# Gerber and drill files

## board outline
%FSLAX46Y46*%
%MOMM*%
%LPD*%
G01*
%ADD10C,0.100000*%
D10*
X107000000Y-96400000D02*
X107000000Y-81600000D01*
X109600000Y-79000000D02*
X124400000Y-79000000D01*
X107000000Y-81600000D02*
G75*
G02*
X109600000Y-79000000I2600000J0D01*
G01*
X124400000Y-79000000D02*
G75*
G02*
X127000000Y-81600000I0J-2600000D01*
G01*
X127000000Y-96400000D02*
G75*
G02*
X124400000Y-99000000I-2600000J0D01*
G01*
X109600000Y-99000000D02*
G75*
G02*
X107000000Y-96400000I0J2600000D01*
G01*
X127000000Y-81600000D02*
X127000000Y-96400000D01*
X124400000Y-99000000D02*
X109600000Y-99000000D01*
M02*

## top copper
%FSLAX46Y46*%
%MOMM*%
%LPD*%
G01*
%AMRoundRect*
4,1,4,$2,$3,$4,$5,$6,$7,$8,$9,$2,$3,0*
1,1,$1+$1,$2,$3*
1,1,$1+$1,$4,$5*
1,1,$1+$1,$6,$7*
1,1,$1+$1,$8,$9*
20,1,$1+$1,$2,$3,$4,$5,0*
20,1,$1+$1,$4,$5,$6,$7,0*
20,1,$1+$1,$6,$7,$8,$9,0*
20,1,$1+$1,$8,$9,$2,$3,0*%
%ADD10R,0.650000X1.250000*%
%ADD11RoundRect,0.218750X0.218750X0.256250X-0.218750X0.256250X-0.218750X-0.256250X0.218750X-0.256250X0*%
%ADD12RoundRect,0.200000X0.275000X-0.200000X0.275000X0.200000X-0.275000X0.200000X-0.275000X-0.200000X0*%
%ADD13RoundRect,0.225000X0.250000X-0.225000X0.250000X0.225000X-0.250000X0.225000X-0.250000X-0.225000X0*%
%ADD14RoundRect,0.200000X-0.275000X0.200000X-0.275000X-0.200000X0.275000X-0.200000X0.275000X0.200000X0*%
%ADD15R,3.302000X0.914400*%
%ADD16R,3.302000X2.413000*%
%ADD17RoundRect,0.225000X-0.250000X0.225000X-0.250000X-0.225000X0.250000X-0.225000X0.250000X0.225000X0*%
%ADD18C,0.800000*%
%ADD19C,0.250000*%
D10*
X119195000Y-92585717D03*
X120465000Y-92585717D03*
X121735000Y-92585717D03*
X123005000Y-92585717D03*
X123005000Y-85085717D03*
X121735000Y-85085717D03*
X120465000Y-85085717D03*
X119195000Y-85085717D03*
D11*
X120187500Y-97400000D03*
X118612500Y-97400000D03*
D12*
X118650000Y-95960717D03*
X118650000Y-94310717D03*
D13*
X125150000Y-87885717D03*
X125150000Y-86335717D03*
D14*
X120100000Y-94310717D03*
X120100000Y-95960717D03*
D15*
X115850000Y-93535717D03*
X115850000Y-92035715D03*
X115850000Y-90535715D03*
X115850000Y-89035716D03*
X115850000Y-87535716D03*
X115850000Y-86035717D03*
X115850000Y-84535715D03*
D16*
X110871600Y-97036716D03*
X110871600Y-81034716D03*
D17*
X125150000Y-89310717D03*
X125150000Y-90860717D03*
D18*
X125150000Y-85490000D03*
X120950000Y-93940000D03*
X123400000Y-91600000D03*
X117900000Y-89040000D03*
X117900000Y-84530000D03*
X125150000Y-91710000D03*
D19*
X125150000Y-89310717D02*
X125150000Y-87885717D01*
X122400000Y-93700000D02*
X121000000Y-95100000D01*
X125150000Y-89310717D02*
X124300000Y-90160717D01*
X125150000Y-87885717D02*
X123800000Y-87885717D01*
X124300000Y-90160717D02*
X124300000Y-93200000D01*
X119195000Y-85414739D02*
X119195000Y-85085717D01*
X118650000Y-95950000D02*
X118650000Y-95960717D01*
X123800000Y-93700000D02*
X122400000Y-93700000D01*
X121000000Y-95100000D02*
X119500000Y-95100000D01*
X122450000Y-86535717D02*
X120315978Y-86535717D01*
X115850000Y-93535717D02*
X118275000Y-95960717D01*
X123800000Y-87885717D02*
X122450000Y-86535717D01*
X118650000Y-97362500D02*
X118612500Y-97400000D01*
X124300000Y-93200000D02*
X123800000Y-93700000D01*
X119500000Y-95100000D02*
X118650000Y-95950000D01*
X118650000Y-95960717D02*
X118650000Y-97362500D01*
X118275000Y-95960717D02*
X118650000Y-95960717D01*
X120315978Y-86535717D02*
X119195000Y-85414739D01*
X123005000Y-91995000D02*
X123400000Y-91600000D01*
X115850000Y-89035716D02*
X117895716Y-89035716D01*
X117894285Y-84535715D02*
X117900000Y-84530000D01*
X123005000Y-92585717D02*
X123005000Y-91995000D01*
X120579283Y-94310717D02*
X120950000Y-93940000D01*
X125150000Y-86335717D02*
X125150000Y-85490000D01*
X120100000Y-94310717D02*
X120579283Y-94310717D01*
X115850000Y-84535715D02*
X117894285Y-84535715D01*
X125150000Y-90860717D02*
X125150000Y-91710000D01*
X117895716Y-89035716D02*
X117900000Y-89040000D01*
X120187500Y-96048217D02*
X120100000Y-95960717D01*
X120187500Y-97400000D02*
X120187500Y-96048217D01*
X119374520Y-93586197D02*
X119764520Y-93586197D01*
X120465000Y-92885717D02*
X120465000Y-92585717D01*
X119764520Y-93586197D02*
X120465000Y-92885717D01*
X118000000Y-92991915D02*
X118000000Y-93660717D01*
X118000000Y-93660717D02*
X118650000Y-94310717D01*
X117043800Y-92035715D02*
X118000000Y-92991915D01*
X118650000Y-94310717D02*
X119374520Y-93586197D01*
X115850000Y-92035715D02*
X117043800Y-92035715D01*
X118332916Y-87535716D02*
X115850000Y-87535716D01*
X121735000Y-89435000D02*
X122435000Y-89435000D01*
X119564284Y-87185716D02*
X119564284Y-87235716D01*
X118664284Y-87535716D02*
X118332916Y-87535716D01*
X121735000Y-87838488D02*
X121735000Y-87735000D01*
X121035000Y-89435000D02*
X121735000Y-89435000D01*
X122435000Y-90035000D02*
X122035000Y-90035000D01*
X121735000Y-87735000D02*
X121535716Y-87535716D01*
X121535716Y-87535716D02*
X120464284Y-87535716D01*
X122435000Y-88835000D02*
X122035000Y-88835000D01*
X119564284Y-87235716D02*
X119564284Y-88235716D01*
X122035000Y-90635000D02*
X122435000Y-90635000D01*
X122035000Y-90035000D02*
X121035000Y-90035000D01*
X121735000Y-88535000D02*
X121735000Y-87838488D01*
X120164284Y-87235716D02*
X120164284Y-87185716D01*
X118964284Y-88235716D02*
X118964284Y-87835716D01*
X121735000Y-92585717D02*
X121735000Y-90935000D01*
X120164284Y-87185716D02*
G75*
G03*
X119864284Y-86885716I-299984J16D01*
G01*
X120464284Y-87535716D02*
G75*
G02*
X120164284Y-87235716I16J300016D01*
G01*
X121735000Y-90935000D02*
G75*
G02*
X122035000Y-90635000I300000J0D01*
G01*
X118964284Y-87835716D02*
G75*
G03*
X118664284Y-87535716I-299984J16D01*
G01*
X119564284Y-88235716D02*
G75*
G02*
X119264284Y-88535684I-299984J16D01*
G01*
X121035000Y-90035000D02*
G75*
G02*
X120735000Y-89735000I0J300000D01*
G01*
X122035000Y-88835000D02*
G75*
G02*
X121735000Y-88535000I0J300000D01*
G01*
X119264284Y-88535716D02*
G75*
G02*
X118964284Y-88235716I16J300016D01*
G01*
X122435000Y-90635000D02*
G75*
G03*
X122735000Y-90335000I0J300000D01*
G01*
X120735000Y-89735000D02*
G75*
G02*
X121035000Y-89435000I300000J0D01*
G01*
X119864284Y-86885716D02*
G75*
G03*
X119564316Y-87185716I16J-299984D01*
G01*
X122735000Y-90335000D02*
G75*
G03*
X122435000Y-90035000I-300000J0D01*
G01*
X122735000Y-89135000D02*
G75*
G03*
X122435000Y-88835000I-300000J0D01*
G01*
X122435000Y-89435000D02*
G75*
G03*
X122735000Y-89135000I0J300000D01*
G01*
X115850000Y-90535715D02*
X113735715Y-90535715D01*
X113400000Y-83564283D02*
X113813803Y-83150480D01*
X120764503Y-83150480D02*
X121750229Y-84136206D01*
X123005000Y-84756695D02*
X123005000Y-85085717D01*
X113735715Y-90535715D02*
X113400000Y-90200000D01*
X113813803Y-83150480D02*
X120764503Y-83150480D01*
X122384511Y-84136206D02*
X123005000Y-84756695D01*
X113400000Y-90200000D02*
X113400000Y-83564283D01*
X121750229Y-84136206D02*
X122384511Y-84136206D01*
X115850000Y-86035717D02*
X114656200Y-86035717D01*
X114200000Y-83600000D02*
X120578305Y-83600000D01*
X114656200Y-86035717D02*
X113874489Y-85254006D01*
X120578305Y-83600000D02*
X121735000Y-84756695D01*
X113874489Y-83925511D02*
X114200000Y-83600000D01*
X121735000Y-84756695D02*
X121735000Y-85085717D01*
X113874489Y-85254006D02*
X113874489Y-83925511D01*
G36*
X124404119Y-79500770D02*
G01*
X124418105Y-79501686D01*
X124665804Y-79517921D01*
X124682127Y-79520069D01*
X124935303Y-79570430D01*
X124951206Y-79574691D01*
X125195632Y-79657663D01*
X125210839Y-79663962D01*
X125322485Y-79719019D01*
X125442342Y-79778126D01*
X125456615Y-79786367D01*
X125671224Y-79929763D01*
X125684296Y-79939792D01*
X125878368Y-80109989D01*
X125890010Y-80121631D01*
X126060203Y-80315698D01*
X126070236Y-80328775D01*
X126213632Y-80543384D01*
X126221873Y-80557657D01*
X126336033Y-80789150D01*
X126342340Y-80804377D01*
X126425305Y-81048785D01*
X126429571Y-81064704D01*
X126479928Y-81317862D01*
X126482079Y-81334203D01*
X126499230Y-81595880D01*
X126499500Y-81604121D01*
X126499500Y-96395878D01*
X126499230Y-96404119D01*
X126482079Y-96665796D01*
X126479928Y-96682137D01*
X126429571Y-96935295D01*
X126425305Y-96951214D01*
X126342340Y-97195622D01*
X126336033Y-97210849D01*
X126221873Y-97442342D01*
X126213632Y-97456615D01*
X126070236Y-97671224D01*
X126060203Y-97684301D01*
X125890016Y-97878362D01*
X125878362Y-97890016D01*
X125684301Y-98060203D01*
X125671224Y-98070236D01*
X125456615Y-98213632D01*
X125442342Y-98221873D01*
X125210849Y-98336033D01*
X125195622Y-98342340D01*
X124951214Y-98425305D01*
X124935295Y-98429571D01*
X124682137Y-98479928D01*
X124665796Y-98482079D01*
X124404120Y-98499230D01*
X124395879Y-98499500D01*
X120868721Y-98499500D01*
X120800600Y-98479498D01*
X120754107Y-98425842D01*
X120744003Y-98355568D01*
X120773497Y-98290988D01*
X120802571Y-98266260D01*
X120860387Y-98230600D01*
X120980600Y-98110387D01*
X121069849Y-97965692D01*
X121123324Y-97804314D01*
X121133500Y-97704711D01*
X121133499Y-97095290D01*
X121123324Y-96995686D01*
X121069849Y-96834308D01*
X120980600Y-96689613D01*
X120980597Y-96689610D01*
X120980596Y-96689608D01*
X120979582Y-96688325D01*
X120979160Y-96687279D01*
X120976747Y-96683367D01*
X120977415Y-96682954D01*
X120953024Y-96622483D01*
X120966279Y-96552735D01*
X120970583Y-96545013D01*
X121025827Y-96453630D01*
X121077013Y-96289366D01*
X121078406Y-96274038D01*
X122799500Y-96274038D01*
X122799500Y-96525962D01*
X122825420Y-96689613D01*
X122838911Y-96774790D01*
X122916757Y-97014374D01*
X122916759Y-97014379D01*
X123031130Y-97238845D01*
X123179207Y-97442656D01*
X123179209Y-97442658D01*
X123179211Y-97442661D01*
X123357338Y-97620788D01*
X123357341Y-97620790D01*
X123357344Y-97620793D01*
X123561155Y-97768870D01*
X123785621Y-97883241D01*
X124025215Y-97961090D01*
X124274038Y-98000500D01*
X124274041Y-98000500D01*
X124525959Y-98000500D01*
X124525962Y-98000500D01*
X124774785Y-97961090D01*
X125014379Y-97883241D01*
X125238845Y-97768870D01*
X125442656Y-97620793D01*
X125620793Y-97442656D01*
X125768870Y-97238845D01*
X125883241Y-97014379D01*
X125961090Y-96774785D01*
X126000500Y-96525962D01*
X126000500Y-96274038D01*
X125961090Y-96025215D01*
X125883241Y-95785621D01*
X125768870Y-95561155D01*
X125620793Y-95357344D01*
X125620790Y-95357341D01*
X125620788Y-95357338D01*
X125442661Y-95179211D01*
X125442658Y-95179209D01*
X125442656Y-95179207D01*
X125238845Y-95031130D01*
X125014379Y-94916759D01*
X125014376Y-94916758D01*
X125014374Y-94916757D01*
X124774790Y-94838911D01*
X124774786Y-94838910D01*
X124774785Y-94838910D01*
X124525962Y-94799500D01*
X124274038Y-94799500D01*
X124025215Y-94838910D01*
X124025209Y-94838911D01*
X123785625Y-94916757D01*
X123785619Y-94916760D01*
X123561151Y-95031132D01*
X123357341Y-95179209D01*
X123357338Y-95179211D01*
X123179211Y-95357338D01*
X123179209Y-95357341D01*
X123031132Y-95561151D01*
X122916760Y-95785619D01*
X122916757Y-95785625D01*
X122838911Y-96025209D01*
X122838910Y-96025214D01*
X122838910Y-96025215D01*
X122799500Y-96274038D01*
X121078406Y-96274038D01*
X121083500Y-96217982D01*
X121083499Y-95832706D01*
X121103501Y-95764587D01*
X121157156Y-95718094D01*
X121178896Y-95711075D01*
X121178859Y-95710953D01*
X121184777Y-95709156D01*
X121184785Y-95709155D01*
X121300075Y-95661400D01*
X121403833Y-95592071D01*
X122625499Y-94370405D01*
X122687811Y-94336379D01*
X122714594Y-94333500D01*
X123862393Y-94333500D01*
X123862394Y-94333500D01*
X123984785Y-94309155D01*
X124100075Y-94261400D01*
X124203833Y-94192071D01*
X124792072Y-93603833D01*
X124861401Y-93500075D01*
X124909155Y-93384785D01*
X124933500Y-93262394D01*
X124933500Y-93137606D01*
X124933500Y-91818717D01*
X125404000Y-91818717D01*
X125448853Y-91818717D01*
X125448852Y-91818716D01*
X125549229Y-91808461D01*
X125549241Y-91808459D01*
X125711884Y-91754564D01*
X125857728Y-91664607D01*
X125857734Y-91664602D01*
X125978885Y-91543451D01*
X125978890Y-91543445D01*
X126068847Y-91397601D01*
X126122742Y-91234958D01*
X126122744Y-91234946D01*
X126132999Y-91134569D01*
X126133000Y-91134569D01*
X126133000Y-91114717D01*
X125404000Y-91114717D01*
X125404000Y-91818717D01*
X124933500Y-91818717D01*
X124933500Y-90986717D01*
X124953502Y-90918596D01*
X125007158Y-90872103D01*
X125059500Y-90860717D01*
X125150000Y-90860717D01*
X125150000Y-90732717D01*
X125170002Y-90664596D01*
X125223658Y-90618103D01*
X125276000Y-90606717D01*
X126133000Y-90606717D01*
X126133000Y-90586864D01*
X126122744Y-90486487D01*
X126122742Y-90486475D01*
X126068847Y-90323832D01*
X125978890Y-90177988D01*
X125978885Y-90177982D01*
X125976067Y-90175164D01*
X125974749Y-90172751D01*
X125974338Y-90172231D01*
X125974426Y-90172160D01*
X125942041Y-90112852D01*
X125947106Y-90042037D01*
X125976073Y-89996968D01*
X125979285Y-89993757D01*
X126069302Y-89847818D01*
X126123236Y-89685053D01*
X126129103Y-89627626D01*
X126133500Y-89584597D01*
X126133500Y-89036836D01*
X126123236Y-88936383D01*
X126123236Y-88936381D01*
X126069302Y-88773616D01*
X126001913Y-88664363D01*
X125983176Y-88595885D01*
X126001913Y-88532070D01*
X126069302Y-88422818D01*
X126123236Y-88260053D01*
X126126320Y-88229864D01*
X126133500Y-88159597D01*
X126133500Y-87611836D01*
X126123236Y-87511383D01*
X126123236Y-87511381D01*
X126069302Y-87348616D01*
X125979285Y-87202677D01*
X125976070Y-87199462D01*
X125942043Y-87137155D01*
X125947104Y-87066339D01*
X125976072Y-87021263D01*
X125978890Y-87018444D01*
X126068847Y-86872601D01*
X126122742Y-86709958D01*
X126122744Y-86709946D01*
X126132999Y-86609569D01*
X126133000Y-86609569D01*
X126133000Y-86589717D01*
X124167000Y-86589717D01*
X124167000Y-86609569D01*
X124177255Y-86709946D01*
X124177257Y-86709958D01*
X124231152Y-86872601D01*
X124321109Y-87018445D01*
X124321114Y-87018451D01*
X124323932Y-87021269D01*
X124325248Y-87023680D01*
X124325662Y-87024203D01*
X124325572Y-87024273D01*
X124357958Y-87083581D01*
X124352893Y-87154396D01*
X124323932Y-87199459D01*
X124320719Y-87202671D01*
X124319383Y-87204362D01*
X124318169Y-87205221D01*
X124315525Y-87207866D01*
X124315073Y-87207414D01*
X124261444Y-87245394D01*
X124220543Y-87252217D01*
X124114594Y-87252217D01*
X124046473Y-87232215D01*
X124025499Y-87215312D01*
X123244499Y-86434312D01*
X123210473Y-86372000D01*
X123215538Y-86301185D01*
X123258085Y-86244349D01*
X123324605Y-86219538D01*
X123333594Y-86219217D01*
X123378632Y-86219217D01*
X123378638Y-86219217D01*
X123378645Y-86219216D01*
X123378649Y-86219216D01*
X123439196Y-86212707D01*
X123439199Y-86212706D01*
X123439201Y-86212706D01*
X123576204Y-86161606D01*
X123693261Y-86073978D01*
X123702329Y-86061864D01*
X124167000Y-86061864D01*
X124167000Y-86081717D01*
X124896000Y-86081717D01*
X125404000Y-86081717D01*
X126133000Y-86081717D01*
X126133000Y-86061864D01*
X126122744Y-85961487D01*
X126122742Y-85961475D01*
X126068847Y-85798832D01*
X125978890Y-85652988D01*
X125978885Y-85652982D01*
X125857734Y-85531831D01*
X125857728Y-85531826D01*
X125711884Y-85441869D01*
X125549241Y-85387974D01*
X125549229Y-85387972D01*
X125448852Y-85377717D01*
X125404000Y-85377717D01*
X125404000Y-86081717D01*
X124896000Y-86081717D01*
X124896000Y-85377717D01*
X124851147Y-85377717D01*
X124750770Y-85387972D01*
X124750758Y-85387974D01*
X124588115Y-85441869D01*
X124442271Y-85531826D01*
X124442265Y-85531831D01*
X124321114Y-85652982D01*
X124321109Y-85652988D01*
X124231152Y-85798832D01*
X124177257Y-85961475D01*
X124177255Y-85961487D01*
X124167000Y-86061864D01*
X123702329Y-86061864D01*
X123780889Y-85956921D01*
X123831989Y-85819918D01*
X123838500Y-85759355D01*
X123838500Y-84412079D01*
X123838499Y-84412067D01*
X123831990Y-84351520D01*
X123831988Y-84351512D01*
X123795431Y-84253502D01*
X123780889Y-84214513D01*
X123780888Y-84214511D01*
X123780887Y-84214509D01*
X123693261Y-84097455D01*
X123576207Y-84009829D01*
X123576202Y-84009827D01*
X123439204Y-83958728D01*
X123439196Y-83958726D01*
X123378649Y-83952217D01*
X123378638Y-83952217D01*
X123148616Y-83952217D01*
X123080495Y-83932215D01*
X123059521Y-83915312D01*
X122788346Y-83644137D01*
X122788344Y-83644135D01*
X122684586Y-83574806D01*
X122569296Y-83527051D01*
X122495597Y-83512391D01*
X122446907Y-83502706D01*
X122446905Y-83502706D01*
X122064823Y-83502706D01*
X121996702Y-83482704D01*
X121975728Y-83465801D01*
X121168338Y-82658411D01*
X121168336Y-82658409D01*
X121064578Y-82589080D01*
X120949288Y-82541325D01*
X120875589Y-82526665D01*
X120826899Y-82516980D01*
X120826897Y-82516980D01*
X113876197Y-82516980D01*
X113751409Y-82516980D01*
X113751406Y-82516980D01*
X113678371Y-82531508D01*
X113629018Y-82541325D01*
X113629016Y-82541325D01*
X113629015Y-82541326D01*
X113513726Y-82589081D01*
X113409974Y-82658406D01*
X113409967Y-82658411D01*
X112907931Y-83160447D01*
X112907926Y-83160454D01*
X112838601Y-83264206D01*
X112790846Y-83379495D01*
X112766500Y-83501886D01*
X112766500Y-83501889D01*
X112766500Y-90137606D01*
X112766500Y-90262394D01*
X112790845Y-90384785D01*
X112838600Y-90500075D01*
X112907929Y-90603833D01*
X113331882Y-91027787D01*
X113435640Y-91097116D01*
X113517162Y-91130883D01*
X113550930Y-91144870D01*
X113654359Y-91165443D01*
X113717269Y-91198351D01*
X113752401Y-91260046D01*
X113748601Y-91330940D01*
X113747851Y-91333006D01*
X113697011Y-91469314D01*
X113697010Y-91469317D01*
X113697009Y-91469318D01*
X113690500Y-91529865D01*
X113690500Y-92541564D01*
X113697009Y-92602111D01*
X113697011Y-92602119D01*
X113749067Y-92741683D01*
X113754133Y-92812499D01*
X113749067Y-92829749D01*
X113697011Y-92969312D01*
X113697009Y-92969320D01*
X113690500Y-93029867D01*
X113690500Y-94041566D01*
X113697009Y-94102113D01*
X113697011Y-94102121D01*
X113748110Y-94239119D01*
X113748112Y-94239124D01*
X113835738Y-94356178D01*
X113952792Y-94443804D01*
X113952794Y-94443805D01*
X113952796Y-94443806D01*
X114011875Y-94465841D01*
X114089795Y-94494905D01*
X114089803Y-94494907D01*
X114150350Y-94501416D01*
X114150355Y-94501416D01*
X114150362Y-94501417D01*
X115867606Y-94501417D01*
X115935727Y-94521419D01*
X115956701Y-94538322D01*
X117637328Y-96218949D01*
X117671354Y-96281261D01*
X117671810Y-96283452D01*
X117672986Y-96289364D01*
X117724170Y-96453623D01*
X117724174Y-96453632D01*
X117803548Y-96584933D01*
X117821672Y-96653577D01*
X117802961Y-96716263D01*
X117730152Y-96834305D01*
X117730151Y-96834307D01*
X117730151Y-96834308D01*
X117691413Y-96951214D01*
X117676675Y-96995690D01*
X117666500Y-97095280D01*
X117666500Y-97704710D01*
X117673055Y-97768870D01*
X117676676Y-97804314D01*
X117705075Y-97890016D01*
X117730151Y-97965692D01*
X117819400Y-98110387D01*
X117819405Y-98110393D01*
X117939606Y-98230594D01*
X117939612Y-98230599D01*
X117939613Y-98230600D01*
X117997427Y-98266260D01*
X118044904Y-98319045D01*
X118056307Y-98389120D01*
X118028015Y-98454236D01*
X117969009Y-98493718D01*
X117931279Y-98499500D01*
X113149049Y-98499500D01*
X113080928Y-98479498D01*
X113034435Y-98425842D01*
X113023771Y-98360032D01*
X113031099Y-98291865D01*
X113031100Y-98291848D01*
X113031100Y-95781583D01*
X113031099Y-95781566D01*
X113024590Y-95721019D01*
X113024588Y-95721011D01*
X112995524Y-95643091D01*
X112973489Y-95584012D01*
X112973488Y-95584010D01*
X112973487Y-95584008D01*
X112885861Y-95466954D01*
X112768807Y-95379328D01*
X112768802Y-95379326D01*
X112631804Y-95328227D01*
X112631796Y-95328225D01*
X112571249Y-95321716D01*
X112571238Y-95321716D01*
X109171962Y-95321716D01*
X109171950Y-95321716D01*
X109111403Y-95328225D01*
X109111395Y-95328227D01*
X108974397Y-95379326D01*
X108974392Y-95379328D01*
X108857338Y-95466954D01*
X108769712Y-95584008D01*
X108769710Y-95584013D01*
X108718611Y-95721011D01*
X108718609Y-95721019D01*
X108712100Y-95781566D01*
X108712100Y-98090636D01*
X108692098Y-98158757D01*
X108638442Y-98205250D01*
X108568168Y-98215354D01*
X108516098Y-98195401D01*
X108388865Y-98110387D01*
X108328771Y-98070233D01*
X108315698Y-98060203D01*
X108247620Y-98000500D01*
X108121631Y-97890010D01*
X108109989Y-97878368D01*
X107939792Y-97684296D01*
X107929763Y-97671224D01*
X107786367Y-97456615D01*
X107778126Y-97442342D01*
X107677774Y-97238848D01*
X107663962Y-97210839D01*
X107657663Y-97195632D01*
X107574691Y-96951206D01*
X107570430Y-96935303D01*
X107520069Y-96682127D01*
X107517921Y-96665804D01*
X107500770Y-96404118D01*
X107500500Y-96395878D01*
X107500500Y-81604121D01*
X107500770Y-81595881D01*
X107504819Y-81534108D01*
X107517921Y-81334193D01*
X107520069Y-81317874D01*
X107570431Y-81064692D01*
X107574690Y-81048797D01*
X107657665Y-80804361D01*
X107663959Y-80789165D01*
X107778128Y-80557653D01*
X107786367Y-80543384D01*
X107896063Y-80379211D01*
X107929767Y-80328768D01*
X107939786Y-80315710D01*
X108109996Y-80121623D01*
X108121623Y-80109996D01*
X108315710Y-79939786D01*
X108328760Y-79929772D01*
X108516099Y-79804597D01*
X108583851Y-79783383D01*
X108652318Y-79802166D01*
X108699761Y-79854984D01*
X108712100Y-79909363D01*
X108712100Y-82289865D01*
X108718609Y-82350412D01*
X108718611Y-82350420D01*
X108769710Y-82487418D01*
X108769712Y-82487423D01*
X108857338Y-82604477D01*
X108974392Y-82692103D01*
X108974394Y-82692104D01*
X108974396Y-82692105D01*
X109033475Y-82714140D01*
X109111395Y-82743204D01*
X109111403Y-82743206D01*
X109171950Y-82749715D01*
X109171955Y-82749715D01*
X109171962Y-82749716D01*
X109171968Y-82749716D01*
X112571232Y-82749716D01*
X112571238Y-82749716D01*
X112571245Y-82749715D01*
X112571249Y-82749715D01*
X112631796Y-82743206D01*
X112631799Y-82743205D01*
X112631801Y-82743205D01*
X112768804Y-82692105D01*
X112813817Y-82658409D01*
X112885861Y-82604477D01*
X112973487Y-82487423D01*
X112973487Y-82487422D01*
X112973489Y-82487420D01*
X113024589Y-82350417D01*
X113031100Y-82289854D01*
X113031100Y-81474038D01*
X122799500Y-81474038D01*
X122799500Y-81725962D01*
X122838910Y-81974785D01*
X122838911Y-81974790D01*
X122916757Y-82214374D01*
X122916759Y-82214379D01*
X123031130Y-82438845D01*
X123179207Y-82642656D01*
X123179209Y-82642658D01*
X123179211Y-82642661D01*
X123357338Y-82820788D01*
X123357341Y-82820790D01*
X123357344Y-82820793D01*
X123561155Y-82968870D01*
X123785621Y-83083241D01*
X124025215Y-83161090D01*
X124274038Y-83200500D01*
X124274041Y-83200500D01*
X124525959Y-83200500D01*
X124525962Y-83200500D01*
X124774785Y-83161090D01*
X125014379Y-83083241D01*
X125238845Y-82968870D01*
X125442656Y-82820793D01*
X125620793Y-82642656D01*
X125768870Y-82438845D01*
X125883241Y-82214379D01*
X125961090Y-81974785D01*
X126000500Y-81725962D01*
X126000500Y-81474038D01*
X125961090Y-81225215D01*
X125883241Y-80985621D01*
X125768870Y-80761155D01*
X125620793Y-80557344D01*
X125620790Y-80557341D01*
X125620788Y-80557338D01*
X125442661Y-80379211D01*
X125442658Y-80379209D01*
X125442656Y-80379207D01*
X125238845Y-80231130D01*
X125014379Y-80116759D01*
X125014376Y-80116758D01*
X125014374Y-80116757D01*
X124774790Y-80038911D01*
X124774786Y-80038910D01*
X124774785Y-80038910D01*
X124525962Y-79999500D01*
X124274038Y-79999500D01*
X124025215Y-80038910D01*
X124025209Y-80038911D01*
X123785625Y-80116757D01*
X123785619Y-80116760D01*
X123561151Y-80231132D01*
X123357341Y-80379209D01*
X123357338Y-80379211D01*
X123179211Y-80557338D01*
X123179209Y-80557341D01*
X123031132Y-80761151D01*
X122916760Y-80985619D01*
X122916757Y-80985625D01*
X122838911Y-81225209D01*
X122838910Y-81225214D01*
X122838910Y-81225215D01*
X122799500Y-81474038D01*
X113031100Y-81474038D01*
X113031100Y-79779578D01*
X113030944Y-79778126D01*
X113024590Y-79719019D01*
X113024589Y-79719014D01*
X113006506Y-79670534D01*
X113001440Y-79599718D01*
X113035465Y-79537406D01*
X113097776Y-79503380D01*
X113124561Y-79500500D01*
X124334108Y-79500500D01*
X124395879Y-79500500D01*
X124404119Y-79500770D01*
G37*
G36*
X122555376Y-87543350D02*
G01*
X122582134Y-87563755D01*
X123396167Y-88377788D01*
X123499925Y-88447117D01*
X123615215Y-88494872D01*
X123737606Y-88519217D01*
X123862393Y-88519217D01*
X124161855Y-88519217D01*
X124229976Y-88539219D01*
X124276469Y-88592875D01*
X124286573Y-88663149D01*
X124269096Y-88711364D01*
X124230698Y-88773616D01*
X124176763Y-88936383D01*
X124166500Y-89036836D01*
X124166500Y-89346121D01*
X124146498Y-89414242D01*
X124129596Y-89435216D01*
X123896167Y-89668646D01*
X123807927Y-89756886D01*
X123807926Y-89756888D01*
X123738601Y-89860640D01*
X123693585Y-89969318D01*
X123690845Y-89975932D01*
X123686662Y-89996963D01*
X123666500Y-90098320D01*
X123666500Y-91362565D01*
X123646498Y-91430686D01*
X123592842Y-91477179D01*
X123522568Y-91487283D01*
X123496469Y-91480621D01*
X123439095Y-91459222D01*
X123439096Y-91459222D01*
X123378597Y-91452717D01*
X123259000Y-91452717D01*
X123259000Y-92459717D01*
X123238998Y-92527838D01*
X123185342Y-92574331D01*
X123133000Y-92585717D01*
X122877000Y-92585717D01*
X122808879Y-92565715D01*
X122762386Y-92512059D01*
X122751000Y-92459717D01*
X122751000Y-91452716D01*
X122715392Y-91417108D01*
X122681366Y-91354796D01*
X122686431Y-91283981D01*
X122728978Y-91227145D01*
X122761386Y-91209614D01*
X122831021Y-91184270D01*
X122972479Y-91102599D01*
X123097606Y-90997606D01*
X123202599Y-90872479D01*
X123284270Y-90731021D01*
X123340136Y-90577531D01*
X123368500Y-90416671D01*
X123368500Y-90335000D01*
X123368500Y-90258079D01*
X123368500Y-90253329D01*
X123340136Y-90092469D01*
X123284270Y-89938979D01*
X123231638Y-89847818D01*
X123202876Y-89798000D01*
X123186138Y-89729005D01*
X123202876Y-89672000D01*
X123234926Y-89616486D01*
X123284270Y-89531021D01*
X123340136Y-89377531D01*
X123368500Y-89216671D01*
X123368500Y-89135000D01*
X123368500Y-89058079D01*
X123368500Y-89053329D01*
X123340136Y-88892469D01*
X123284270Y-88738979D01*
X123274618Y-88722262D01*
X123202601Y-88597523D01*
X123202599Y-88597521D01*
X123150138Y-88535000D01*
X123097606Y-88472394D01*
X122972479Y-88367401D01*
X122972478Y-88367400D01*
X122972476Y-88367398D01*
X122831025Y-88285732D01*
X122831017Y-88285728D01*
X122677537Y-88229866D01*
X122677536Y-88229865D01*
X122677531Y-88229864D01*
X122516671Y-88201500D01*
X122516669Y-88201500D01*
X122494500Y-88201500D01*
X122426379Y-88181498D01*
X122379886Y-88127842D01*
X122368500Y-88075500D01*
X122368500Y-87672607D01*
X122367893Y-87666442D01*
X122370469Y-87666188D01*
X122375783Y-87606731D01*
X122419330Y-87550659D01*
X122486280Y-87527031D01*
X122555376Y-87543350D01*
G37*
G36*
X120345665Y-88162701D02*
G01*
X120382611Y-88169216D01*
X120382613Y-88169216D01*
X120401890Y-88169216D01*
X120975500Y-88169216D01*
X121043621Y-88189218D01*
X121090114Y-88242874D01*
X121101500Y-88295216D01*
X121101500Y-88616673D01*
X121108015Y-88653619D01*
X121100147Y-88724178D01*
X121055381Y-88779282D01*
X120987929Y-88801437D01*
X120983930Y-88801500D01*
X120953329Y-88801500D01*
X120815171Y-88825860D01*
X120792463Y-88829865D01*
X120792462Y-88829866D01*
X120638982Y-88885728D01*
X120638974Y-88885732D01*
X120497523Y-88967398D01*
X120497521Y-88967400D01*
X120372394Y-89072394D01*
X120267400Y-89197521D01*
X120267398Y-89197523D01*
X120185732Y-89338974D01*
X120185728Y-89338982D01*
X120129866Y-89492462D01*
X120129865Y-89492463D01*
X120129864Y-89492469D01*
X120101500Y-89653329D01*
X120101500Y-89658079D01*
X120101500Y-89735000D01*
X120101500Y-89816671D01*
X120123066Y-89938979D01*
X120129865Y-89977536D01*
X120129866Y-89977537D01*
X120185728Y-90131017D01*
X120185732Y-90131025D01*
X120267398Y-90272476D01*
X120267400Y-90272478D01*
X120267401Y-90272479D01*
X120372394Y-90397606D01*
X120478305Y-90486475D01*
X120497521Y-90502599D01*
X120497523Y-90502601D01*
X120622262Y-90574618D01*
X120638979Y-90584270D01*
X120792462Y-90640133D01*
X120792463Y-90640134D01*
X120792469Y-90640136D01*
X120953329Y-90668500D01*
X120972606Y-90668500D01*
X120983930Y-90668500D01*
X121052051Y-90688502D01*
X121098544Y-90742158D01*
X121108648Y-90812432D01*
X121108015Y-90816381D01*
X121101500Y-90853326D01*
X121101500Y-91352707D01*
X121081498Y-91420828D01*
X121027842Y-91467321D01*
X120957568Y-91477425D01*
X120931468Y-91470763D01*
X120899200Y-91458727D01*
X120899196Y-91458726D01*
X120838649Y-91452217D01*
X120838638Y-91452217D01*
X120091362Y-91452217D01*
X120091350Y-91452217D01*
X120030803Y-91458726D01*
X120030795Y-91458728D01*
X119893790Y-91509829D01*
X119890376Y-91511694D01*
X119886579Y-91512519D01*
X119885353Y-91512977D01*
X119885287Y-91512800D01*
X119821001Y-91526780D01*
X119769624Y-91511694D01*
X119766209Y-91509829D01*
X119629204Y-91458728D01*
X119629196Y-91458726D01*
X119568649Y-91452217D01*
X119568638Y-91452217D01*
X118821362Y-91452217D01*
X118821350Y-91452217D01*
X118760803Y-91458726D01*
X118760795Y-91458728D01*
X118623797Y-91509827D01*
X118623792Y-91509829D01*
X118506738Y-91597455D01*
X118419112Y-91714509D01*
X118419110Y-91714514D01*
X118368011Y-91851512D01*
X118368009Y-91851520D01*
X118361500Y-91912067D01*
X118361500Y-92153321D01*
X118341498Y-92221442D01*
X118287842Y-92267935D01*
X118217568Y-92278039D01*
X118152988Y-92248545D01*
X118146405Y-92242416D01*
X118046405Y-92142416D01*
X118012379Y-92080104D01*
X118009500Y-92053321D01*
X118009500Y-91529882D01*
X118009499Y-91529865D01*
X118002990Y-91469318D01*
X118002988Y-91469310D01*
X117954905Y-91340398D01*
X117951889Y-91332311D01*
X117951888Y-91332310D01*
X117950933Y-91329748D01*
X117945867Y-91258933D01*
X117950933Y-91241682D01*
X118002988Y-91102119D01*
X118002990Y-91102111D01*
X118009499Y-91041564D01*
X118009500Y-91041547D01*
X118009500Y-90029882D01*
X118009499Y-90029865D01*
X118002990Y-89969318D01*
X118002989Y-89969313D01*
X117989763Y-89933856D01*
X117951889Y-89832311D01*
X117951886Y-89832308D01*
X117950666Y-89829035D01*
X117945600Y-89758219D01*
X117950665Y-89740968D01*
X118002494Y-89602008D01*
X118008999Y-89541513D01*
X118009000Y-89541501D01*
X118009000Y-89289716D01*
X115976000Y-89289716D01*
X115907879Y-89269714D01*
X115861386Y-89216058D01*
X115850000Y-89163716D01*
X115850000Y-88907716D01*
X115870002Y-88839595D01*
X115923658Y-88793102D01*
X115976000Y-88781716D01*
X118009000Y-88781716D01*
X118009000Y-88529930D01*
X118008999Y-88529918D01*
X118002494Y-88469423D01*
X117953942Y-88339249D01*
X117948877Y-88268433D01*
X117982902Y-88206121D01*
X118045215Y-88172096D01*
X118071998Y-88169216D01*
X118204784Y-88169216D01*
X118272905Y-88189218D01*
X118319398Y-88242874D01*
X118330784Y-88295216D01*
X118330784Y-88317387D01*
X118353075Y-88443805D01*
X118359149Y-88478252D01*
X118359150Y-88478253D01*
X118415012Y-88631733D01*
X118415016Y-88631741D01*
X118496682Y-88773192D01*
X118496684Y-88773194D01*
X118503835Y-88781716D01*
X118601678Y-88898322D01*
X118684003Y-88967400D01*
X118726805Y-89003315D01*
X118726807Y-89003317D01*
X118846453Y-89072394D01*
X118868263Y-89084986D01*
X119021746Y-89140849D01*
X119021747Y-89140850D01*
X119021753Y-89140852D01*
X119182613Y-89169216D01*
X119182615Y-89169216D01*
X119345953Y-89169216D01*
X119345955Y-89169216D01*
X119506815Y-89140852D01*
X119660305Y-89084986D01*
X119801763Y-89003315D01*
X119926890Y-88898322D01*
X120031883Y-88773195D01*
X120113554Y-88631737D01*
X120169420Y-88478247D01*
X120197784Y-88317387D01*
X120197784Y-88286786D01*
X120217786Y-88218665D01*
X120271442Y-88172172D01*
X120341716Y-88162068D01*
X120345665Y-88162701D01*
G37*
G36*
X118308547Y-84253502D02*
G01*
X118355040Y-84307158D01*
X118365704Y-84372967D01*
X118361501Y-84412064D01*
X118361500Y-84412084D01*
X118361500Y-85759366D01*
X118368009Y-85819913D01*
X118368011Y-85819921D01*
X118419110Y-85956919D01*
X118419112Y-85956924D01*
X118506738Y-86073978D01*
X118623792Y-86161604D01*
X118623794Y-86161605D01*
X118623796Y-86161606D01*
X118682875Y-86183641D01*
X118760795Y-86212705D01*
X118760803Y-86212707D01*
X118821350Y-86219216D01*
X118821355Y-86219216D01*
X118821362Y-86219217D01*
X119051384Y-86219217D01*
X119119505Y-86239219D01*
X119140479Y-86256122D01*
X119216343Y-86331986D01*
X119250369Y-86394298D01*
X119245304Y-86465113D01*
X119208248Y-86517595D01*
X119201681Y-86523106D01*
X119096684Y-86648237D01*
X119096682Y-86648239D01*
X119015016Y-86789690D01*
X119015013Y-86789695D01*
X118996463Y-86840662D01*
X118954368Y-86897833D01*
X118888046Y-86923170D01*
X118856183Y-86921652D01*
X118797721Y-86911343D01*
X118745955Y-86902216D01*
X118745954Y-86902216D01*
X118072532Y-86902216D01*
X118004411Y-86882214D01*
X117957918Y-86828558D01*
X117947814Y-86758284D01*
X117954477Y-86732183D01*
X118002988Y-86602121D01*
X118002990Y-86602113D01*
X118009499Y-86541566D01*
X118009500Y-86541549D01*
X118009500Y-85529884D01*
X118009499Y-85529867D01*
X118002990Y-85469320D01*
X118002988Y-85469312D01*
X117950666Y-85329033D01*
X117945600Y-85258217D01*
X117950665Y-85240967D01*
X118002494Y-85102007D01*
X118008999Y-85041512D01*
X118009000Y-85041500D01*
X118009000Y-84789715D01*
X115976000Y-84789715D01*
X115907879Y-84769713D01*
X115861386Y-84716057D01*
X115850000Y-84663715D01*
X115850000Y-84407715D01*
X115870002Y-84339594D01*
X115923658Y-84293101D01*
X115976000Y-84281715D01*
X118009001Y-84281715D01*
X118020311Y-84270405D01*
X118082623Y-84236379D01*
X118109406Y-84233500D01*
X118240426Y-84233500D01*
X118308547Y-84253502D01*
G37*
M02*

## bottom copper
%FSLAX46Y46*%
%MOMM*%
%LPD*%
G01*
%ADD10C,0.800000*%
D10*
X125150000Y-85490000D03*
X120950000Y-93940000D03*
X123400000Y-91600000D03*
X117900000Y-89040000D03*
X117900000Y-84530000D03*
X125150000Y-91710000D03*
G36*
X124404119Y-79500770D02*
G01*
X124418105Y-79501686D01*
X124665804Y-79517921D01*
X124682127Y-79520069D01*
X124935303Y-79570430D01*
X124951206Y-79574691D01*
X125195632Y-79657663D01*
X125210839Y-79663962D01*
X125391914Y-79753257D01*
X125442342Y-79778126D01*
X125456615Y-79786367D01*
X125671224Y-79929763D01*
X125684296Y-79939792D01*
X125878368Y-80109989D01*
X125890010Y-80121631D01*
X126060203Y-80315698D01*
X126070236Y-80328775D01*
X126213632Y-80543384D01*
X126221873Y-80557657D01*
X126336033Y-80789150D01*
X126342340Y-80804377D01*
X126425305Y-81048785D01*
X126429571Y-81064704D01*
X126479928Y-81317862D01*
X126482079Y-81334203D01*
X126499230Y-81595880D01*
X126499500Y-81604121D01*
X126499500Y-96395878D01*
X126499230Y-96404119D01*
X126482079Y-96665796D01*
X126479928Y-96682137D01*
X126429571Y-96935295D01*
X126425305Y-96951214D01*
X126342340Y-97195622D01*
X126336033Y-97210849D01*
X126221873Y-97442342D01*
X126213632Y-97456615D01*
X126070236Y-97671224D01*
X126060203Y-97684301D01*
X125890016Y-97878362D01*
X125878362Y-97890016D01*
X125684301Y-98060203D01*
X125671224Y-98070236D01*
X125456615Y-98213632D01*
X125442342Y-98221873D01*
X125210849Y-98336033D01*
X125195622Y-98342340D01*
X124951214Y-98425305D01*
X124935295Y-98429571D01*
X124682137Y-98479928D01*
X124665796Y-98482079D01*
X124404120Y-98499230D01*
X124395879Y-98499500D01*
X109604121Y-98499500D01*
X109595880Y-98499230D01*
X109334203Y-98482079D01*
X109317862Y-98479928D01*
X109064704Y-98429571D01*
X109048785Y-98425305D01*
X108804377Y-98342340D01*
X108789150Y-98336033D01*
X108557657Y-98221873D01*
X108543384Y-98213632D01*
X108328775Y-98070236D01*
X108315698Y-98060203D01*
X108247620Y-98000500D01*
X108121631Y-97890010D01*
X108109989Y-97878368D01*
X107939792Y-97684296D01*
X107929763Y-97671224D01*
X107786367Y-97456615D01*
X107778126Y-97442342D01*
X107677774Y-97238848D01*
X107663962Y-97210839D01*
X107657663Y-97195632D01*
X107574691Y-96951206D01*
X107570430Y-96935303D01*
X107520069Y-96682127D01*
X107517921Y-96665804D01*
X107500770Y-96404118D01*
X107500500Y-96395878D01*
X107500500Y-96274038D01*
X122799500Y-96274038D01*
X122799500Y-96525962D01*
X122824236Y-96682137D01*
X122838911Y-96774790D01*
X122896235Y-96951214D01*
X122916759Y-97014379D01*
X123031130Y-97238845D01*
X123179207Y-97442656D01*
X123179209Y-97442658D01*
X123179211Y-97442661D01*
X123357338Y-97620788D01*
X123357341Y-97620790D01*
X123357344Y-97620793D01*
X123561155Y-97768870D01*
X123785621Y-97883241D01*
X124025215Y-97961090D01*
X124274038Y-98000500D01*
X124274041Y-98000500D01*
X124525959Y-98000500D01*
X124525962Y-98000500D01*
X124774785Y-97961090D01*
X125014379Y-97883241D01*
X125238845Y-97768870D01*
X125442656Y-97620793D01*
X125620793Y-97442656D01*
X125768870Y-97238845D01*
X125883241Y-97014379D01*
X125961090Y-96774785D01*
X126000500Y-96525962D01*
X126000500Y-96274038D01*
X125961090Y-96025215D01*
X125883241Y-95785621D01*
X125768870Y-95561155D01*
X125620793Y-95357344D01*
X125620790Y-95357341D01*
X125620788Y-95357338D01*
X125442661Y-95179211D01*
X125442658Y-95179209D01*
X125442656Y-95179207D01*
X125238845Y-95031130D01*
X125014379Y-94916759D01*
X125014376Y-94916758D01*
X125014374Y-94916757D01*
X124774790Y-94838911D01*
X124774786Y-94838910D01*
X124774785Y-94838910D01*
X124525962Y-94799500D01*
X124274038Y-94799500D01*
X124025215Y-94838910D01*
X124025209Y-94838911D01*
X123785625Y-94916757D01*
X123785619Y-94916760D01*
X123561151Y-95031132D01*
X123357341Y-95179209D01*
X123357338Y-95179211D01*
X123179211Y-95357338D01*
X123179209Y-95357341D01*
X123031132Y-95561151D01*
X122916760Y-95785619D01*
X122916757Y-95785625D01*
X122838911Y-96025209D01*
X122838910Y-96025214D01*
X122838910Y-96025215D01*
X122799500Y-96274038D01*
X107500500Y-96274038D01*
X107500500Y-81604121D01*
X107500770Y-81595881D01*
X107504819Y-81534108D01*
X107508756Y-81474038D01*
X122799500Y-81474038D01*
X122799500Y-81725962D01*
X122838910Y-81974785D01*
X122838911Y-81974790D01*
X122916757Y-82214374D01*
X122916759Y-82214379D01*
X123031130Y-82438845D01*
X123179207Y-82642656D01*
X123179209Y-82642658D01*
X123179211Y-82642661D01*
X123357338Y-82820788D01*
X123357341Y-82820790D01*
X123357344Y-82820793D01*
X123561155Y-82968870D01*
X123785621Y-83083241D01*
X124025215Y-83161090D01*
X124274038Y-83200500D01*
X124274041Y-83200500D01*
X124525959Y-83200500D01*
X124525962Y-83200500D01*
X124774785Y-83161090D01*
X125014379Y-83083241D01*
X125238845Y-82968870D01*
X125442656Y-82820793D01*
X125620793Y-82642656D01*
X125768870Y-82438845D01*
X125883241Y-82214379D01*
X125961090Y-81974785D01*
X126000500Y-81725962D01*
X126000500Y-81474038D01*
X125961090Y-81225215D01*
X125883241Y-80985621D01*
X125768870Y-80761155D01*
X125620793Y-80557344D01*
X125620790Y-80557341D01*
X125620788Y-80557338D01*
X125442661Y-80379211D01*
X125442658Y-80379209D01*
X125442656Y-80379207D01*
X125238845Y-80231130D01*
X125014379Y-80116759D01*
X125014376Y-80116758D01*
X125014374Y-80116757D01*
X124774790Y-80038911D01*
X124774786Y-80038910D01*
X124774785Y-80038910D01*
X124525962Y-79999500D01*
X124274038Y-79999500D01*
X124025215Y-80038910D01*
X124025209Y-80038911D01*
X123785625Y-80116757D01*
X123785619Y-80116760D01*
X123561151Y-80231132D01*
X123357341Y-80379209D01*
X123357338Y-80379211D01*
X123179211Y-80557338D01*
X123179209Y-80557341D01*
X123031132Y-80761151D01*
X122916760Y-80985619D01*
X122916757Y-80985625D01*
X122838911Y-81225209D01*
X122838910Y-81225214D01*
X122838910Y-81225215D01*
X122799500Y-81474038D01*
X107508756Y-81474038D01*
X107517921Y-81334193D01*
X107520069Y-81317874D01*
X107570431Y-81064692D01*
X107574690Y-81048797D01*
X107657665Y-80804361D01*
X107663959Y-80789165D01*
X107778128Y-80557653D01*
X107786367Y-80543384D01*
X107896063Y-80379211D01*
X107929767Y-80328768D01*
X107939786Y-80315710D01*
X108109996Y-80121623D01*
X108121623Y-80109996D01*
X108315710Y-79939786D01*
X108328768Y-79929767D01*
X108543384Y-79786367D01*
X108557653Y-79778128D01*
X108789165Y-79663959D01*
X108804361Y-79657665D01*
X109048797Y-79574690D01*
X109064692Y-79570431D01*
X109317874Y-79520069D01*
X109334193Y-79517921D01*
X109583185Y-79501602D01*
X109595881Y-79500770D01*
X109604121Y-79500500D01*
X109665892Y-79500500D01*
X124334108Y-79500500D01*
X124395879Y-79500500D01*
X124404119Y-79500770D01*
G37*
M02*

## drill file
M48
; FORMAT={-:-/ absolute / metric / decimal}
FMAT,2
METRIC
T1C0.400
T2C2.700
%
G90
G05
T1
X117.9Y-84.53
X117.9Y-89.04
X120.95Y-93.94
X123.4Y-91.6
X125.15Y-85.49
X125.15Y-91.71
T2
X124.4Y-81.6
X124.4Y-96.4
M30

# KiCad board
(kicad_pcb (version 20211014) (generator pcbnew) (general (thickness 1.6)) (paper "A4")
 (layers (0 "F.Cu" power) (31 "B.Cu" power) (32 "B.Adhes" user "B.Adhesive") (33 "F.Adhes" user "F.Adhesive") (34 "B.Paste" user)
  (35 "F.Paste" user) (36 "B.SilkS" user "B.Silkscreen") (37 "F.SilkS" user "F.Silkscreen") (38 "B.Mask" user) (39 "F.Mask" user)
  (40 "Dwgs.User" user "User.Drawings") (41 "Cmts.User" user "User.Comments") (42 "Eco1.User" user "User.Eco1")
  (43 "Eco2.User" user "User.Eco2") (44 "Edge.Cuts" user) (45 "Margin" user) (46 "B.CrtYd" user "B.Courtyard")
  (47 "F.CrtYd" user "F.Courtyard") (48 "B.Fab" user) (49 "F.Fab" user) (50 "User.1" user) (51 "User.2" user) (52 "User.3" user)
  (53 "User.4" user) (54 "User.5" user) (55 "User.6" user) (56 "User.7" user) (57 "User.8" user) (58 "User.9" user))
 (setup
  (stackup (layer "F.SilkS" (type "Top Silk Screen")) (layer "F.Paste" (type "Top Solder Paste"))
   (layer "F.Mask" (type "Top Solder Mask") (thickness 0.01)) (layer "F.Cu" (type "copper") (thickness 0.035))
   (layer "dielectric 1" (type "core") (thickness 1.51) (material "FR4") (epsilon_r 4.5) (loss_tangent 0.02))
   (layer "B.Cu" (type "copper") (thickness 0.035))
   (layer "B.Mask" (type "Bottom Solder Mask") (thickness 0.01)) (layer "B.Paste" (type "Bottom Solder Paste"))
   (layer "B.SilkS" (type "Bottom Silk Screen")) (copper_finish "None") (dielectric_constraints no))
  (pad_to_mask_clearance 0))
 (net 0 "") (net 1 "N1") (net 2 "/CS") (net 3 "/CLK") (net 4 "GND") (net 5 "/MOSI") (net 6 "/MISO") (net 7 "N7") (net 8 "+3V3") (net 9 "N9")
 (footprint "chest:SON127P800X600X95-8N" (layer "F.Cu") (at 121.1 88.835717 90)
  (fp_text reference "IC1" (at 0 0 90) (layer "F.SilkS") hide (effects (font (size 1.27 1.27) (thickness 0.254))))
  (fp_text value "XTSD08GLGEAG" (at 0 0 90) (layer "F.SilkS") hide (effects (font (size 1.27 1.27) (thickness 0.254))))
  (pad "1" smd rect (at -3.75 -1.905 180) (size 0.65 1.25) (layers "F.Cu" "F.Paste" "F.Mask") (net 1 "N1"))
  (pad "2" smd rect (at -3.75 -0.635 180) (size 0.65 1.25) (layers "F.Cu" "F.Paste" "F.Mask") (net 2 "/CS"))
  (pad "3" smd rect (at -3.75 0.635 180) (size 0.65 1.25) (layers "F.Cu" "F.Paste" "F.Mask") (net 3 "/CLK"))
  (pad "4" smd rect (at -3.75 1.905 180) (size 0.65 1.25) (layers "F.Cu" "F.Paste" "F.Mask") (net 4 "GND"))
  (pad "5" smd rect (at 3.75 1.905 180) (size 0.65 1.25) (layers "F.Cu" "F.Paste" "F.Mask") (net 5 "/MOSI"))
  (pad "6" smd rect (at 3.75 0.635 180) (size 0.65 1.25) (layers "F.Cu" "F.Paste" "F.Mask") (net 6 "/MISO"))
  (pad "7" smd rect (at 3.75 -0.635 180) (size 0.65 1.25) (layers "F.Cu" "F.Paste" "F.Mask") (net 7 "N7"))
  (pad "8" smd rect (at 3.75 -1.905 180) (size 0.65 1.25) (layers "F.Cu" "F.Paste" "F.Mask") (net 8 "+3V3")))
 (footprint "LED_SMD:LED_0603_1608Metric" (layer "F.Cu") (at 119.4 97.4 180)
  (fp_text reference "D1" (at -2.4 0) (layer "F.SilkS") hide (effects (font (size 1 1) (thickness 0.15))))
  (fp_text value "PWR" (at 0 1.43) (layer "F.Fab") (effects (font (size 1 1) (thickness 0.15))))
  (pad "1" smd roundrect (at -0.7875 0 180) (size 0.875 0.95) (layers "F.Cu" "F.Paste" "F.Mask") (roundrect_rratio 0.25) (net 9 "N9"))
  (pad "2" smd roundrect (at 0.7875 0 180) (size 0.875 0.95) (layers "F.Cu" "F.Paste" "F.Mask") (roundrect_rratio 0.25) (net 8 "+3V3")))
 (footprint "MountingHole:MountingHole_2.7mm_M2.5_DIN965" (layer "F.Cu") (at 124.4 81.6)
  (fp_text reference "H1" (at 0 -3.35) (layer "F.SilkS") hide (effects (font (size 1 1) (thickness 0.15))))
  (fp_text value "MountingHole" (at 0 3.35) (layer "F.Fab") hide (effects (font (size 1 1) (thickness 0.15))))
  (pad "" np_thru_hole circle (at 0 0) (size 2.7 2.7) (drill 2.7) (layers *.Cu *.Mask)))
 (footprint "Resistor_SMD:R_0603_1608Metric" (layer "F.Cu") (at 118.65 95.135717 90)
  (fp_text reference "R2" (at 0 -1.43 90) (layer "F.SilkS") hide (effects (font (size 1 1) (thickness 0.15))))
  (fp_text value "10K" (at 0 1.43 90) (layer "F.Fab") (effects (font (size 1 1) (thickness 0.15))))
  (pad "1" smd roundrect (at -0.825 0 90) (size 0.8 0.95) (layers "F.Cu" "F.Paste" "F.Mask") (roundrect_rratio 0.25) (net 8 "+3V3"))
  (pad "2" smd roundrect (at 0.825 0 90) (size 0.8 0.95) (layers "F.Cu" "F.Paste" "F.Mask") (roundrect_rratio 0.25) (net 2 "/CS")))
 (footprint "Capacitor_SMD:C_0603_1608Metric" (layer "F.Cu") (at 125.15 87.110717 90)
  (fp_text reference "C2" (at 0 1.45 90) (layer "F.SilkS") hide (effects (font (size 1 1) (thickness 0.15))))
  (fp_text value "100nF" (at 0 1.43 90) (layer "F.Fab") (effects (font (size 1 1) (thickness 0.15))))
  (pad "1" smd roundrect (at -0.775 0 90) (size 0.9 0.95) (layers "F.Cu" "F.Paste" "F.Mask") (roundrect_rratio 0.25) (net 8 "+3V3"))
  (pad "2" smd roundrect (at 0.775 0 90) (size 0.9 0.95) (layers "F.Cu" "F.Paste" "F.Mask") (roundrect_rratio 0.25) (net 4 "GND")))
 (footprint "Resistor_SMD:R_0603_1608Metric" (layer "F.Cu") (at 120.1 95.135717 -90)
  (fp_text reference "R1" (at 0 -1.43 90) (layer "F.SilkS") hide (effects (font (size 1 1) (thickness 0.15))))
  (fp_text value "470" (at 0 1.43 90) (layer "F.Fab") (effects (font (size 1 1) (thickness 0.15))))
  (pad "1" smd roundrect (at -0.825 0 270) (size 0.8 0.95) (layers "F.Cu" "F.Paste" "F.Mask") (roundrect_rratio 0.25) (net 4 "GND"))
  (pad "2" smd roundrect (at 0.825 0 270) (size 0.8 0.95) (layers "F.Cu" "F.Paste" "F.Mask") (roundrect_rratio 0.25) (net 9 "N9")))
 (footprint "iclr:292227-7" (layer "F.Cu") (at 115.85 93.535717 90)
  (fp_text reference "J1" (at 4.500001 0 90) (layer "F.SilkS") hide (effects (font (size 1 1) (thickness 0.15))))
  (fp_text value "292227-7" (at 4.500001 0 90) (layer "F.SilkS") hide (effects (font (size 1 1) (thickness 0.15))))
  (pad "1" smd rect (at 0 0 90) (size 0.9144 3.302) (layers "F.Cu" "F.Paste" "F.Mask") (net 8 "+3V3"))
  (pad "2" smd rect (at 1.500002 0 90) (size 0.9144 3.302) (layers "F.Cu" "F.Paste" "F.Mask") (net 2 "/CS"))
  (pad "3" smd rect (at 3.000002 0 90) (size 0.9144 3.302) (layers "F.Cu" "F.Paste" "F.Mask") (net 5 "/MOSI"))
  (pad "4" smd rect (at 4.500001 0 90) (size 0.9144 3.302) (layers "F.Cu" "F.Paste" "F.Mask") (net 4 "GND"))
  (pad "5" smd rect (at 6.000001 0 90) (size 0.9144 3.302) (layers "F.Cu" "F.Paste" "F.Mask") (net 3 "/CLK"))
  (pad "6" smd rect (at 7.5 0 90) (size 0.9144 3.302) (layers "F.Cu" "F.Paste" "F.Mask") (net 6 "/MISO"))
  (pad "7" smd rect (at 9.000002 0 90) (size 0.9144 3.302) (layers "F.Cu" "F.Paste" "F.Mask") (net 4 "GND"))
  (pad "8" smd rect (at -3.500999 -4.9784 90) (size 2.413 3.302) (layers "F.Cu" "F.Paste" "F.Mask"))
  (pad "9" smd rect (at 12.501001 -4.9784 90) (size 2.413 3.302) (layers "F.Cu" "F.Paste" "F.Mask")))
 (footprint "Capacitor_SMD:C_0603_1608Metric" (layer "F.Cu") (at 125.15 90.085717 -90)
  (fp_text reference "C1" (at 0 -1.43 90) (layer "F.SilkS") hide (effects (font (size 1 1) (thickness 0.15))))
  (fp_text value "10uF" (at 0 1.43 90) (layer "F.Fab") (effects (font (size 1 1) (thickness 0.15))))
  (pad "1" smd roundrect (at -0.775 0 270) (size 0.9 0.95) (layers "F.Cu" "F.Paste" "F.Mask") (roundrect_rratio 0.25) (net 8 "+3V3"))
  (pad "2" smd roundrect (at 0.775 0 270) (size 0.9 0.95) (layers "F.Cu" "F.Paste" "F.Mask") (roundrect_rratio 0.25) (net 4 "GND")))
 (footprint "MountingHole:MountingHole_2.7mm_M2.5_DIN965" (layer "F.Cu") (at 124.4 96.4)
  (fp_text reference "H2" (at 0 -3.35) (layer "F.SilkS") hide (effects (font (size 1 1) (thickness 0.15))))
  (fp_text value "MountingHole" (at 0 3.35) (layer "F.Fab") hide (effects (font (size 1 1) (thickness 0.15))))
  (pad "" np_thru_hole circle (at 0 0) (size 2.7 2.7) (drill 2.7) (layers *.Cu *.Mask)))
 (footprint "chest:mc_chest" (layer "B.Cu") (at 113.4 88.8 -90)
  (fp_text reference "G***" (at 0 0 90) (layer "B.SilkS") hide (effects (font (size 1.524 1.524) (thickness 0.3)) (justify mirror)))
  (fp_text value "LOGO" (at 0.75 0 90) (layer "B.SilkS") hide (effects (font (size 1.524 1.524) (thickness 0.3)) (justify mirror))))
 (gr_line (start 107 96.4) (end 107 81.6) (layer "Edge.Cuts") (width 0.1))
 (gr_line (start 109.6 79) (end 124.4 79) (layer "Edge.Cuts") (width 0.1))
 (gr_arc (start 107 81.6) (mid 107.761522 79.761522) (end 109.6 79) (layer "Edge.Cuts") (width 0.1))
 (gr_arc (start 124.4 79) (mid 126.238478 79.761522) (end 127 81.6) (layer "Edge.Cuts") (width 0.1))
 (gr_arc (start 127 96.4) (mid 126.238478 98.238478) (end 124.4 99) (layer "Edge.Cuts") (width 0.1))
 (gr_arc (start 109.6 99) (mid 107.761522 98.238478) (end 107 96.4) (layer "Edge.Cuts") (width 0.1))
 (gr_line (start 127 81.6) (end 127 96.4) (layer "Edge.Cuts") (width 0.1))
 (gr_line (start 124.4 99) (end 109.6 99) (layer "Edge.Cuts") (width 0.1))
 (segment (start 125.15 89.310717) (end 125.15 87.885717) (width 0.25) (layer "F.Cu") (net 8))
 (segment (start 122.4 93.7) (end 121 95.1) (width 0.25) (layer "F.Cu") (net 8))
 (segment (start 125.15 89.310717) (end 124.3 90.160717) (width 0.25) (layer "F.Cu") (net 8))
 (segment (start 125.15 87.885717) (end 123.8 87.885717) (width 0.25) (layer "F.Cu") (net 8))
 (segment (start 124.3 90.160717) (end 124.3 93.2) (width 0.25) (layer "F.Cu") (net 8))
 (segment (start 119.195 85.414739) (end 119.195 85.085717) (width 0.25) (layer "F.Cu") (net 8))
 (segment (start 118.65 95.95) (end 118.65 95.960717) (width 0.25) (layer "F.Cu") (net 8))
 (segment (start 123.8 93.7) (end 122.4 93.7) (width 0.25) (layer "F.Cu") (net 8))
 (segment (start 121 95.1) (end 119.5 95.1) (width 0.25) (layer "F.Cu") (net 8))
 (segment (start 122.45 86.535717) (end 120.315978 86.535717) (width 0.25) (layer "F.Cu") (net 8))
 (segment (start 115.85 93.535717) (end 118.275 95.960717) (width 0.25) (layer "F.Cu") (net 8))
 (segment (start 123.8 87.885717) (end 122.45 86.535717) (width 0.25) (layer "F.Cu") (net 8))
 (segment (start 118.65 97.3625) (end 118.6125 97.4) (width 0.25) (layer "F.Cu") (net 8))
 (segment (start 124.3 93.2) (end 123.8 93.7) (width 0.25) (layer "F.Cu") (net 8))
 (segment (start 119.5 95.1) (end 118.65 95.95) (width 0.25) (layer "F.Cu") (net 8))
 (segment (start 118.65 95.960717) (end 118.65 97.3625) (width 0.25) (layer "F.Cu") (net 8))
 (segment (start 118.275 95.960717) (end 118.65 95.960717) (width 0.25) (layer "F.Cu") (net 8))
 (segment (start 120.315978 86.535717) (end 119.195 85.414739) (width 0.25) (layer "F.Cu") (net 8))
 (segment (start 123.005 91.995) (end 123.4 91.6) (width 0.25) (layer "F.Cu") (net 4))
 (segment (start 115.85 89.035716) (end 117.895716 89.035716) (width 0.25) (layer "F.Cu") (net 4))
 (segment (start 117.894285 84.535715) (end 117.9 84.53) (width 0.25) (layer "F.Cu") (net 4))
 (segment (start 123.005 92.585717) (end 123.005 91.995) (width 0.25) (layer "F.Cu") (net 4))
 (segment (start 120.579283 94.310717) (end 120.95 93.94) (width 0.25) (layer "F.Cu") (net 4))
 (segment (start 125.15 86.335717) (end 125.15 85.49) (width 0.25) (layer "F.Cu") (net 4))
 (segment (start 120.1 94.310717) (end 120.579283 94.310717) (width 0.25) (layer "F.Cu") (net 4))
 (segment (start 115.85 84.535715) (end 117.894285 84.535715) (width 0.25) (layer "F.Cu") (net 4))
 (segment (start 125.15 90.860717) (end 125.15 91.71) (width 0.25) (layer "F.Cu") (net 4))
 (segment (start 117.895716 89.035716) (end 117.9 89.04) (width 0.25) (layer "F.Cu") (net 4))
 (via (at 125.15 85.49) (size 0.8) (drill 0.4) (layers "F.Cu" "B.Cu") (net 4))
 (via (at 120.95 93.94) (size 0.8) (drill 0.4) (layers "F.Cu" "B.Cu") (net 4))
 (via (at 123.4 91.6) (size 0.8) (drill 0.4) (layers "F.Cu" "B.Cu") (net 4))
 (via (at 117.9 89.04) (size 0.8) (drill 0.4) (layers "F.Cu" "B.Cu") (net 4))
 (via (at 117.9 84.53) (size 0.8) (drill 0.4) (layers "F.Cu" "B.Cu") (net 4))
 (via (at 125.15 91.71) (size 0.8) (drill 0.4) (layers "F.Cu" "B.Cu") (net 4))
 (segment (start 120.1875 96.048217) (end 120.1 95.960717) (width 0.25) (layer "F.Cu") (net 9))
 (segment (start 120.1875 97.4) (end 120.1875 96.048217) (width 0.25) (layer "F.Cu") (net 9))
 (segment (start 119.37452 93.586197) (end 119.76452 93.586197) (width 0.25) (layer "F.Cu") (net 2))
 (segment (start 120.465 92.885717) (end 120.465 92.585717) (width 0.25) (layer "F.Cu") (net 2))
 (segment (start 119.76452 93.586197) (end 120.465 92.885717) (width 0.25) (layer "F.Cu") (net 2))
 (segment (start 118 92.991915) (end 118 93.660717) (width 0.25) (layer "F.Cu") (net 2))
 (segment (start 118 93.660717) (end 118.65 94.310717) (width 0.25) (layer "F.Cu") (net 2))
 (segment (start 117.0438 92.035715) (end 118 92.991915) (width 0.25) (layer "F.Cu") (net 2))
 (segment (start 118.65 94.310717) (end 119.37452 93.586197) (width 0.25) (layer "F.Cu") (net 2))
 (segment (start 115.85 92.035715) (end 117.0438 92.035715) (width 0.25) (layer "F.Cu") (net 2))
 (segment (start 118.332916 87.535716) (end 115.85 87.535716) (width 0.25) (layer "F.Cu") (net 3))
 (segment (start 121.735 89.435) (end 122.435 89.435) (width 0.25) (layer "F.Cu") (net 3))
 (segment (start 119.564284 87.185716) (end 119.564284 87.235716) (width 0.25) (layer "F.Cu") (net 3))
 (segment (start 118.664284 87.535716) (end 118.332916 87.535716) (width 0.25) (layer "F.Cu") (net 3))
 (segment (start 121.735 87.838488) (end 121.735 87.735) (width 0.25) (layer "F.Cu") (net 3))
 (segment (start 121.035 89.435) (end 121.735 89.435) (width 0.25) (layer "F.Cu") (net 3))
 (segment (start 122.435 90.035) (end 122.035 90.035) (width 0.25) (layer "F.Cu") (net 3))
 (segment (start 121.735 87.735) (end 121.535716 87.535716) (width 0.25) (layer "F.Cu") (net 3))
 (segment (start 121.535716 87.535716) (end 120.464284 87.535716) (width 0.25) (layer "F.Cu") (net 3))
 (segment (start 122.435 88.835) (end 122.035 88.835) (width 0.25) (layer "F.Cu") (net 3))
 (segment (start 119.564284 87.235716) (end 119.564284 88.235716) (width 0.25) (layer "F.Cu") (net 3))
 (segment (start 122.035 90.635) (end 122.435 90.635) (width 0.25) (layer "F.Cu") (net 3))
 (segment (start 122.035 90.035) (end 121.035 90.035) (width 0.25) (layer "F.Cu") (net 3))
 (segment (start 121.735 88.535) (end 121.735 87.838488) (width 0.25) (layer "F.Cu") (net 3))
 (segment (start 120.164284 87.235716) (end 120.164284 87.185716) (width 0.25) (layer "F.Cu") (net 3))
 (segment (start 118.964284 88.235716) (end 118.964284 87.835716) (width 0.25) (layer "F.Cu") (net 3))
 (segment (start 121.735 92.585717) (end 121.735 90.935) (width 0.25) (layer "F.Cu") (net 3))
 (arc (start 120.164284 87.185716) (mid 120.076416 86.973584) (end 119.864284 86.885716) (width 0.25) (layer "F.Cu") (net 3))
 (arc (start 120.464284 87.535716) (mid 120.252152 87.447848) (end 120.164284 87.235716) (width 0.25) (layer "F.Cu") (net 3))
 (arc (start 121.735 90.935) (mid 121.822868 90.722868) (end 122.035 90.635) (width 0.25) (layer "F.Cu") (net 3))
 (arc (start 118.964284 87.835716) (mid 118.876416 87.623584) (end 118.664284 87.535716) (width 0.25) (layer "F.Cu") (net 3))
 (arc (start 119.564284 88.235716) (mid 119.476416 88.447848) (end 119.264284 88.535716) (width 0.25) (layer "F.Cu") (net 3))
 (arc (start 121.035 90.035) (mid 120.822868 89.947132) (end 120.735 89.735) (width 0.25) (layer "F.Cu") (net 3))
 (arc (start 122.035 88.835) (mid 121.822868 88.747132) (end 121.735 88.535) (width 0.25) (layer "F.Cu") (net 3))
 (arc (start 119.264284 88.535716) (mid 119.052152 88.447848) (end 118.964284 88.235716) (width 0.25) (layer "F.Cu") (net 3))
 (arc (start 122.435 90.635) (mid 122.647132 90.547132) (end 122.735 90.335) (width 0.25) (layer "F.Cu") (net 3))
 (arc (start 120.735 89.735) (mid 120.822868 89.522868) (end 121.035 89.435) (width 0.25) (layer "F.Cu") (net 3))
 (arc (start 119.864284 86.885716) (mid 119.652152 86.973584) (end 119.564284 87.185716) (width 0.25) (layer "F.Cu") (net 3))
 (arc (start 122.735 90.335) (mid 122.647132 90.122868) (end 122.435 90.035) (width 0.25) (layer "F.Cu") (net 3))
 (arc (start 122.735 89.135) (mid 122.647132 88.922868) (end 122.435 88.835) (width 0.25) (layer "F.Cu") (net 3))
 (arc (start 122.435 89.435) (mid 122.647132 89.347132) (end 122.735 89.135) (width 0.25) (layer "F.Cu") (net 3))
 (segment (start 115.85 90.535715) (end 113.735715 90.535715) (width 0.25) (layer "F.Cu") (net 5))
 (segment (start 113.4 83.564283) (end 113.813803 83.15048) (width 0.25) (layer "F.Cu") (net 5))
 (segment (start 120.764503 83.15048) (end 121.750229 84.136206) (width 0.25) (layer "F.Cu") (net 5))
 (segment (start 123.005 84.756695) (end 123.005 85.085717) (width 0.25) (layer "F.Cu") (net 5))
 (segment (start 113.735715 90.535715) (end 113.4 90.2) (width 0.25) (layer "F.Cu") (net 5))
 (segment (start 113.813803 83.15048) (end 120.764503 83.15048) (width 0.25) (layer "F.Cu") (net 5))
 (segment (start 122.384511 84.136206) (end 123.005 84.756695) (width 0.25) (layer "F.Cu") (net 5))
 (segment (start 113.4 90.2) (end 113.4 83.564283) (width 0.25) (layer "F.Cu") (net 5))
 (segment (start 121.750229 84.136206) (end 122.384511 84.136206) (width 0.25) (layer "F.Cu") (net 5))
 (segment (start 115.85 86.035717) (end 114.6562 86.035717) (width 0.25) (layer "F.Cu") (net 6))
 (segment (start 114.2 83.6) (end 120.578305 83.6) (width 0.25) (layer "F.Cu") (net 6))
 (segment (start 114.6562 86.035717) (end 113.874489 85.254006) (width 0.25) (layer "F.Cu") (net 6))
 (segment (start 120.578305 83.6) (end 121.735 84.756695) (width 0.25) (layer "F.Cu") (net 6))
 (segment (start 113.874489 83.925511) (end 114.2 83.6) (width 0.25) (layer "F.Cu") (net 6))
 (segment (start 121.735 84.756695) (end 121.735 85.085717) (width 0.25) (layer "F.Cu") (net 6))
 (segment (start 113.874489 85.254006) (end 113.874489 83.925511) (width 0.25) (layer "F.Cu") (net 6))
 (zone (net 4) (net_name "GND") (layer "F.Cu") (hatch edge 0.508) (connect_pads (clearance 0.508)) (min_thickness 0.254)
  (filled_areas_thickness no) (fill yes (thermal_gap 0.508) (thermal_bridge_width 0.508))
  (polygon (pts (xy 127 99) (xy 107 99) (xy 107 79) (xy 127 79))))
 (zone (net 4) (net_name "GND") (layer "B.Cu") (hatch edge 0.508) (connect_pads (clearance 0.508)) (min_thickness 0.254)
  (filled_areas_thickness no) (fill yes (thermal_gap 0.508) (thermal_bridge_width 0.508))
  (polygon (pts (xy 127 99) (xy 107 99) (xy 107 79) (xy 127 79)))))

